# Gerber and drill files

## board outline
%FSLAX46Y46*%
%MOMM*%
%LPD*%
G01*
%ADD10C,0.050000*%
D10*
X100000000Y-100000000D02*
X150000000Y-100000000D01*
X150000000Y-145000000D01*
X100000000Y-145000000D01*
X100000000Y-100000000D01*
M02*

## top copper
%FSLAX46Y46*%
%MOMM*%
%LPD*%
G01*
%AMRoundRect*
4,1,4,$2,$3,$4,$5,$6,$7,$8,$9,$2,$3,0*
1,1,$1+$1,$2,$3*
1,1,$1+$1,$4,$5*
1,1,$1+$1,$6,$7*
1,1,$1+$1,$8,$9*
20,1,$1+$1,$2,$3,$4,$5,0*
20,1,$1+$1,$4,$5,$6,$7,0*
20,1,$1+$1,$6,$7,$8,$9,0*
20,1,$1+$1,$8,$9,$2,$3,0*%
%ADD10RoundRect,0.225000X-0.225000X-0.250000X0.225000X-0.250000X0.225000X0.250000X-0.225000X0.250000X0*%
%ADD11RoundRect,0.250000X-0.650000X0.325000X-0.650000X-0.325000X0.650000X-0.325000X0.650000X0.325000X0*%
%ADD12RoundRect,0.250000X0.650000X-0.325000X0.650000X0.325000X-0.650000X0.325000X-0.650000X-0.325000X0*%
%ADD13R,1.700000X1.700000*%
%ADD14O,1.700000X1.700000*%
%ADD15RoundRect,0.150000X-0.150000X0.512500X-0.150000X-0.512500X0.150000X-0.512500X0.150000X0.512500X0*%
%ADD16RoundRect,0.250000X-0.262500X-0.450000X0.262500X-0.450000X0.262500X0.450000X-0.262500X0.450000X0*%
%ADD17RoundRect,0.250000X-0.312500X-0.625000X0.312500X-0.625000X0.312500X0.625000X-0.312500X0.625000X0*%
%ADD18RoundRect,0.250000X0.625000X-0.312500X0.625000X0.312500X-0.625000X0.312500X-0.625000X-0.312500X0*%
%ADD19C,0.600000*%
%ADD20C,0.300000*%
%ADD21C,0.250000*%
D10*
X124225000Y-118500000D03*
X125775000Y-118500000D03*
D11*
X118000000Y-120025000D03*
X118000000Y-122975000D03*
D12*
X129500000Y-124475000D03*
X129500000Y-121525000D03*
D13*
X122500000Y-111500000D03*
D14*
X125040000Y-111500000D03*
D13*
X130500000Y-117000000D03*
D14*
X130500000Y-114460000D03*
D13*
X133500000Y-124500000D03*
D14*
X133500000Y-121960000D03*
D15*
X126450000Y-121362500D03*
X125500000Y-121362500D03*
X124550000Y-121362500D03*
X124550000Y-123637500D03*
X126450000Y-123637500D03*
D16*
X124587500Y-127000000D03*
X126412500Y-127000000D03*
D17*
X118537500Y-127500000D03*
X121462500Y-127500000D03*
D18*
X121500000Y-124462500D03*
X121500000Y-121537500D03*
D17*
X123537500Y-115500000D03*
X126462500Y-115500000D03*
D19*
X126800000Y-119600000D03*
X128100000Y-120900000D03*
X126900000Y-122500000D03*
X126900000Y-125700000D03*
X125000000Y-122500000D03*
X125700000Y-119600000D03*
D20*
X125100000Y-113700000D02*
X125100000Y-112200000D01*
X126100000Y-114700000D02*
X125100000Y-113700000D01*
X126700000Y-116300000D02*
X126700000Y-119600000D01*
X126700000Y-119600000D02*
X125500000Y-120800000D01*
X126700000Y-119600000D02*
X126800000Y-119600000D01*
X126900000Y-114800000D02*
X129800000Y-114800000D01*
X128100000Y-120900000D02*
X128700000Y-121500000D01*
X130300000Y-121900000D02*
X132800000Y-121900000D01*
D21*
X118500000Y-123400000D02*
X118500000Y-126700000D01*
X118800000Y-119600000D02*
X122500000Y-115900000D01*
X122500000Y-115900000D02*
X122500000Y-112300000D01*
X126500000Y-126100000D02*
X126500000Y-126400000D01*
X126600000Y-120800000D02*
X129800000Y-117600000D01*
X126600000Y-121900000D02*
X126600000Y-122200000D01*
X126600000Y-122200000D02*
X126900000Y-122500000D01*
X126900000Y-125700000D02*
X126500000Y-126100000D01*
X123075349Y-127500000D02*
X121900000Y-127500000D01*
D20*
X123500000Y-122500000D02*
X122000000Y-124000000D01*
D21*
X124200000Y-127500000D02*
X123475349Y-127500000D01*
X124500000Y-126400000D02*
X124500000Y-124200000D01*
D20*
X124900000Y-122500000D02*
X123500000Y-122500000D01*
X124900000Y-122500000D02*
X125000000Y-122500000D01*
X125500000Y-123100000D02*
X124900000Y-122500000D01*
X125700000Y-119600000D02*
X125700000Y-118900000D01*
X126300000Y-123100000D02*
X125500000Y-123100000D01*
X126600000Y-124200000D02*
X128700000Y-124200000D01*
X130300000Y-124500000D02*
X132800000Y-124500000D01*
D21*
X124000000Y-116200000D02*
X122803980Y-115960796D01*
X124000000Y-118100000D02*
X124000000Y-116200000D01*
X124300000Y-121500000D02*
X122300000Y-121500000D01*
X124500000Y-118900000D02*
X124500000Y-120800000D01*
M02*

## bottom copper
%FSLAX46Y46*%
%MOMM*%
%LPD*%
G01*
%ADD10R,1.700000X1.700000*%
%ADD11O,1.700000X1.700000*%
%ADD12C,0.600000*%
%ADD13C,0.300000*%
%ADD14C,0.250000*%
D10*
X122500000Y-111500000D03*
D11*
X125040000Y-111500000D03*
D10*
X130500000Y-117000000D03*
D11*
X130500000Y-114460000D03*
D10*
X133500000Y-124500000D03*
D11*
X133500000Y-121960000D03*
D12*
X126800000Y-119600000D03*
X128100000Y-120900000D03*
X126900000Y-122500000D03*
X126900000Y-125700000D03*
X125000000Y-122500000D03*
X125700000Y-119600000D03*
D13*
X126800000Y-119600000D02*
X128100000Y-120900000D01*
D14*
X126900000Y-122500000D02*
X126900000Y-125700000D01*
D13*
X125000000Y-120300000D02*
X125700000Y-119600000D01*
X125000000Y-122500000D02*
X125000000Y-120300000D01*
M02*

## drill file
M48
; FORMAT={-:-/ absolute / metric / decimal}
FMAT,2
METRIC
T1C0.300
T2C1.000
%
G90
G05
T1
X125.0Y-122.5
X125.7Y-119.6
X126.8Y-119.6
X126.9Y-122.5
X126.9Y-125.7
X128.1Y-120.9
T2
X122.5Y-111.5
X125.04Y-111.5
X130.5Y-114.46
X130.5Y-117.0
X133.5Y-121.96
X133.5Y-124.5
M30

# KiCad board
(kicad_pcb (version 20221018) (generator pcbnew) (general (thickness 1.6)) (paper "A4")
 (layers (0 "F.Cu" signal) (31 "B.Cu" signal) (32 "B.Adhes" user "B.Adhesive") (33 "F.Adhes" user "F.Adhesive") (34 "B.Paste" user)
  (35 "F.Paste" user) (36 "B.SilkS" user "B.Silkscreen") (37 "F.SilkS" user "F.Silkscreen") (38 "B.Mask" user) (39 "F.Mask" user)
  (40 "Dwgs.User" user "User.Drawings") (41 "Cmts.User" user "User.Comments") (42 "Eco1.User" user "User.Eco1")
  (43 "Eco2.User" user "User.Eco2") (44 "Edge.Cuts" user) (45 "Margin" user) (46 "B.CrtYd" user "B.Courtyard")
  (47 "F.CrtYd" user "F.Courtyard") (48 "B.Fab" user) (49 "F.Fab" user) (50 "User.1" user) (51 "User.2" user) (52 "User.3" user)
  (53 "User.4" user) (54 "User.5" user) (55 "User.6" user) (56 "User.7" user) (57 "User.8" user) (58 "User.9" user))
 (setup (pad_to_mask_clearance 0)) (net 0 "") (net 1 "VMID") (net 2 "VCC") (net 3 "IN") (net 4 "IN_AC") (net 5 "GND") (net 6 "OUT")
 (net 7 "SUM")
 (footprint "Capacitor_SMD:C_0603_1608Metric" (layer "F.Cu") (at 125 118.5)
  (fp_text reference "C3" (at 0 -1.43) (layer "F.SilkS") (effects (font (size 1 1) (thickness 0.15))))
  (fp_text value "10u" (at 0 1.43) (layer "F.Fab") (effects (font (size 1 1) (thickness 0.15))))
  (pad "1" smd roundrect (at -0.775 0) (size 0.9 0.95) (layers "F.Cu" "F.Paste" "F.Mask") (roundrect_rratio 0.25) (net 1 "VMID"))
  (pad "2" smd roundrect (at 0.775 0) (size 0.9 0.95) (layers "F.Cu" "F.Paste" "F.Mask") (roundrect_rratio 0.25) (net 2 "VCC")))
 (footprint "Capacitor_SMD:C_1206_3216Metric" (layer "F.Cu") (at 118 121.5 -90)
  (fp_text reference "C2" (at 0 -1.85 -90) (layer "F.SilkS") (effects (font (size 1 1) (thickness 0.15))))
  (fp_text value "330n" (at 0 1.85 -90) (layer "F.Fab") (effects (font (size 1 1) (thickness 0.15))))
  (pad "1" smd roundrect (at -1.475 0 270) (size 1.15 1.8) (layers "F.Cu" "F.Paste" "F.Mask") (roundrect_rratio 0.217391) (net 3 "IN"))
  (pad "2" smd roundrect (at 1.475 0 270) (size 1.15 1.8) (layers "F.Cu" "F.Paste" "F.Mask") (roundrect_rratio 0.217391) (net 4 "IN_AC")))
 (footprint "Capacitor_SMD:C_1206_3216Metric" (layer "F.Cu") (at 129.5 123 90)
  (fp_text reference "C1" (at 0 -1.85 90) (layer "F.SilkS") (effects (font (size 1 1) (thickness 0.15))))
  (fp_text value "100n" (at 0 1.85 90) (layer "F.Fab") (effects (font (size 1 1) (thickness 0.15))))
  (pad "1" smd roundrect (at -1.475 0 90) (size 1.15 1.8) (layers "F.Cu" "F.Paste" "F.Mask") (roundrect_rratio 0.217391) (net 2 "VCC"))
  (pad "2" smd roundrect (at 1.475 0 90) (size 1.15 1.8) (layers "F.Cu" "F.Paste" "F.Mask") (roundrect_rratio 0.217391) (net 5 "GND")))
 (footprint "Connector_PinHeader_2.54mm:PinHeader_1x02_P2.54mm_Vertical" (layer "F.Cu") (at 122.5 111.5 90)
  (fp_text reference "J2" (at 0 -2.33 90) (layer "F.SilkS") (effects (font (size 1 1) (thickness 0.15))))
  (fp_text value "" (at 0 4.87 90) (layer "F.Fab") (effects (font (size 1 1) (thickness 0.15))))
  (pad "1" thru_hole rect (at 0 0 90) (size 1.7 1.7) (drill 1) (layers "*.Cu" "*.Mask") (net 3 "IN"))
  (pad "2" thru_hole oval (at 0 2.54 90) (size 1.7 1.7) (drill 1) (layers "*.Cu" "*.Mask") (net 5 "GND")))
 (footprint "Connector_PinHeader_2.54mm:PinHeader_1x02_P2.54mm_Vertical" (layer "F.Cu") (at 130.5 117 180)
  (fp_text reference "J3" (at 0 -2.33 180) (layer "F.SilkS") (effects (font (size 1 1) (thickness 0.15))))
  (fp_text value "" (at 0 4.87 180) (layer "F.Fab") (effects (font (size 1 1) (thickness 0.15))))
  (pad "1" thru_hole rect (at 0 0 180) (size 1.7 1.7) (drill 1) (layers "*.Cu" "*.Mask") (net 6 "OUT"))
  (pad "2" thru_hole oval (at 0 2.54 180) (size 1.7 1.7) (drill 1) (layers "*.Cu" "*.Mask") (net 5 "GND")))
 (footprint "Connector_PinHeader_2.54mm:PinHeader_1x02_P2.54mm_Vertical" (layer "F.Cu") (at 133.5 124.5 180)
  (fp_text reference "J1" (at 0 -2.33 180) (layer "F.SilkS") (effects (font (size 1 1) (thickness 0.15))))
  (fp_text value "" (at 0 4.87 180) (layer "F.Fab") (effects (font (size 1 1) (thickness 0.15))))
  (pad "1" thru_hole rect (at 0 0 180) (size 1.7 1.7) (drill 1) (layers "*.Cu" "*.Mask") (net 2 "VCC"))
  (pad "2" thru_hole oval (at 0 2.54 180) (size 1.7 1.7) (drill 1) (layers "*.Cu" "*.Mask") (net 5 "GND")))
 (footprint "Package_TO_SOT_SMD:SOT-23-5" (layer "F.Cu") (at 125.5 122.5 -90)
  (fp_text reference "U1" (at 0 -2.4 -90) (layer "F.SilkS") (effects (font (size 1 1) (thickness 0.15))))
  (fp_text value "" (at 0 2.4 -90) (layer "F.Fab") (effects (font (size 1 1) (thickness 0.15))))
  (pad "1" smd roundrect (at -1.1375 -0.95 270) (size 1.325 0.6) (layers "F.Cu" "F.Paste" "F.Mask") (roundrect_rratio 0.25) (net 6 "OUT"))
  (pad "2" smd roundrect (at -1.1375 0 270) (size 1.325 0.6) (layers "F.Cu" "F.Paste" "F.Mask") (roundrect_rratio 0.25) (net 5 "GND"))
  (pad "3" smd roundrect (at -1.1375 0.95 270) (size 1.325 0.6) (layers "F.Cu" "F.Paste" "F.Mask") (roundrect_rratio 0.25) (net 1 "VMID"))
  (pad "4" smd roundrect (at 1.1375 0.95 270) (size 1.325 0.6) (layers "F.Cu" "F.Paste" "F.Mask") (roundrect_rratio 0.25) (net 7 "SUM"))
  (pad "5" smd roundrect (at 1.1375 -0.95 270) (size 1.325 0.6) (layers "F.Cu" "F.Paste" "F.Mask") (roundrect_rratio 0.25) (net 2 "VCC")))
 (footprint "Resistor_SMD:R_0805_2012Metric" (layer "F.Cu") (at 125.5 127)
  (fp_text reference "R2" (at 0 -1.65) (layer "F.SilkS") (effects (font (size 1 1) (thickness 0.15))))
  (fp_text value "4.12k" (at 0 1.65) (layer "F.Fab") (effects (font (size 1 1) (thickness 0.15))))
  (pad "1" smd roundrect (at -0.9125 0) (size 1.025 1.4) (layers "F.Cu" "F.Paste" "F.Mask") (roundrect_rratio 0.243902) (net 7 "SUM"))
  (pad "2" smd roundrect (at 0.9125 0) (size 1.025 1.4) (layers "F.Cu" "F.Paste" "F.Mask") (roundrect_rratio 0.243902) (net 6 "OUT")))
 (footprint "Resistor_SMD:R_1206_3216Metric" (layer "F.Cu") (at 120 127.5)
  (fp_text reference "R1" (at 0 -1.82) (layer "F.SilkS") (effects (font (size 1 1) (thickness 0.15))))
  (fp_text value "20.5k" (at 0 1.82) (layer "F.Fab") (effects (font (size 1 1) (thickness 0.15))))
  (pad "1" smd roundrect (at -1.4625 0) (size 1.125 1.75) (layers "F.Cu" "F.Paste" "F.Mask") (roundrect_rratio 0.222222) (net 4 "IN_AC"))
  (pad "2" smd roundrect (at 1.4625 0) (size 1.125 1.75) (layers "F.Cu" "F.Paste" "F.Mask") (roundrect_rratio 0.222222) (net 7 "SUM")))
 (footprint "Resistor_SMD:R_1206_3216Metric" (layer "F.Cu") (at 121.5 123 90)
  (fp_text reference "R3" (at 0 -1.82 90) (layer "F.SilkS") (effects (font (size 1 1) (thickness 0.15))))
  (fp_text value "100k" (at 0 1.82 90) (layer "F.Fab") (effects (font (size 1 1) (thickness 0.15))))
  (pad "1" smd roundrect (at -1.4625 0 90) (size 1.125 1.75) (layers "F.Cu" "F.Paste" "F.Mask") (roundrect_rratio 0.222222) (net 2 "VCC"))
  (pad "2" smd roundrect (at 1.4625 0 90) (size 1.125 1.75) (layers "F.Cu" "F.Paste" "F.Mask") (roundrect_rratio 0.222222) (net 1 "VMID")))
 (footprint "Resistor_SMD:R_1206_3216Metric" (layer "F.Cu") (at 125 115.5)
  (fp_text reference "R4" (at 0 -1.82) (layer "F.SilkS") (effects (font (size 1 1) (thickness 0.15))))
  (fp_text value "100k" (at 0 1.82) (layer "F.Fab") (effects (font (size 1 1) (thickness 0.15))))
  (pad "1" smd roundrect (at -1.4625 0) (size 1.125 1.75) (layers "F.Cu" "F.Paste" "F.Mask") (roundrect_rratio 0.222222) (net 1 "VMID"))
  (pad "2" smd roundrect (at 1.4625 0) (size 1.125 1.75) (layers "F.Cu" "F.Paste" "F.Mask") (roundrect_rratio 0.222222) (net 5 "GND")))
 (gr_rect (start 100 100) (end 150 145) (stroke (width 0.05) (type default)) (fill none) (layer "Edge.Cuts"))
 (segment (start 125.1 113.7) (end 125.1 112.2) (width 0.3) (layer "F.Cu") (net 5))
 (segment (start 126.1 114.7) (end 125.1 113.7) (width 0.3) (layer "F.Cu") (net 5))
 (segment (start 126.7 116.3) (end 126.7 119.6) (width 0.3) (layer "F.Cu") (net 5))
 (segment (start 126.7 119.6) (end 125.5 120.8) (width 0.3) (layer "F.Cu") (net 5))
 (segment (start 126.7 119.6) (end 126.8 119.6) (width 0.3) (layer "F.Cu") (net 5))
 (segment (start 126.9 114.8) (end 129.8 114.8) (width 0.3) (layer "F.Cu") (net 5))
 (segment (start 128.1 120.9) (end 128.7 121.5) (width 0.3) (layer "F.Cu") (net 5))
 (segment (start 130.3 121.9) (end 132.8 121.9) (width 0.3) (layer "F.Cu") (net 5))
 (via (at 126.8 119.6) (size 0.6) (drill 0.3) (layers "F.Cu" "B.Cu") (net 5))
 (via (at 128.1 120.9) (size 0.6) (drill 0.3) (layers "F.Cu" "B.Cu") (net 5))
 (segment (start 118.5 123.4) (end 118.5 126.7) (width 0.25) (layer "F.Cu") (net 4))
 (segment (start 118.8 119.6) (end 122.5 115.9) (width 0.25) (layer "F.Cu") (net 3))
 (segment (start 122.5 115.9) (end 122.5 112.3) (width 0.25) (layer "F.Cu") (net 3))
 (segment (start 126.5 126.1) (end 126.5 126.4) (width 0.25) (layer "F.Cu") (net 6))
 (segment (start 126.6 120.8) (end 129.8 117.6) (width 0.25) (layer "F.Cu") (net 6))
 (segment (start 126.6 121.9) (end 126.6 122.2) (width 0.25) (layer "F.Cu") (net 6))
 (segment (start 126.6 122.2) (end 126.9 122.5) (width 0.25) (layer "F.Cu") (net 6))
 (segment (start 126.8 119.6) (end 128.1 120.9) (width 0.3) (layer "B.Cu") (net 5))
 (segment (start 126.9 125.7) (end 126.5 126.1) (width 0.25) (layer "F.Cu") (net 6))
 (via (at 126.9 122.5) (size 0.6) (drill 0.3) (layers "F.Cu" "B.Cu") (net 6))
 (via (at 126.9 125.7) (size 0.6) (drill 0.3) (layers "F.Cu" "B.Cu") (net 6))
 (segment (start 123.075349 127.5) (end 121.9 127.5) (width 0.25) (layer "F.Cu") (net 7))
 (segment (start 123.5 122.5) (end 122 124) (width 0.3) (layer "F.Cu") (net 2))
 (segment (start 124.2 127.5) (end 123.475349 127.5) (width 0.25) (layer "F.Cu") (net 7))
 (segment (start 124.5 126.4) (end 124.5 124.2) (width 0.25) (layer "F.Cu") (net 7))
 (segment (start 124.9 122.5) (end 123.5 122.5) (width 0.3) (layer "F.Cu") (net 2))
 (segment (start 124.9 122.5) (end 125 122.5) (width 0.3) (layer "F.Cu") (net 2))
 (segment (start 125.5 123.1) (end 124.9 122.5) (width 0.3) (layer "F.Cu") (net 2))
 (segment (start 125.7 119.6) (end 125.7 118.9) (width 0.3) (layer "F.Cu") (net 2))
 (segment (start 126.3 123.1) (end 125.5 123.1) (width 0.3) (layer "F.Cu") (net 2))
 (segment (start 126.6 124.2) (end 128.7 124.2) (width 0.3) (layer "F.Cu") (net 2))
 (segment (start 126.9 122.5) (end 126.9 125.7) (width 0.25) (layer "B.Cu") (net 6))
 (segment (start 130.3 124.5) (end 132.8 124.5) (width 0.3) (layer "F.Cu") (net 2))
 (via (at 125 122.5) (size 0.6) (drill 0.3) (layers "F.Cu" "B.Cu") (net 2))
 (via (at 125.7 119.6) (size 0.6) (drill 0.3) (layers "F.Cu" "B.Cu") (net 2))
 (segment (start 124 116.2) (end 122.80398 115.960796) (width 0.25) (layer "F.Cu") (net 1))
 (segment (start 124 118.1) (end 124 116.2) (width 0.25) (layer "F.Cu") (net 1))
 (segment (start 124.3 121.5) (end 122.3 121.5) (width 0.25) (layer "F.Cu") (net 1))
 (segment (start 124.5 118.9) (end 124.5 120.8) (width 0.25) (layer "F.Cu") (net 1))
 (segment (start 125 120.3) (end 125.7 119.6) (width 0.3) (layer "B.Cu") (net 2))
 (segment (start 125 122.5) (end 125 120.3) (width 0.3) (layer "B.Cu") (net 2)))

